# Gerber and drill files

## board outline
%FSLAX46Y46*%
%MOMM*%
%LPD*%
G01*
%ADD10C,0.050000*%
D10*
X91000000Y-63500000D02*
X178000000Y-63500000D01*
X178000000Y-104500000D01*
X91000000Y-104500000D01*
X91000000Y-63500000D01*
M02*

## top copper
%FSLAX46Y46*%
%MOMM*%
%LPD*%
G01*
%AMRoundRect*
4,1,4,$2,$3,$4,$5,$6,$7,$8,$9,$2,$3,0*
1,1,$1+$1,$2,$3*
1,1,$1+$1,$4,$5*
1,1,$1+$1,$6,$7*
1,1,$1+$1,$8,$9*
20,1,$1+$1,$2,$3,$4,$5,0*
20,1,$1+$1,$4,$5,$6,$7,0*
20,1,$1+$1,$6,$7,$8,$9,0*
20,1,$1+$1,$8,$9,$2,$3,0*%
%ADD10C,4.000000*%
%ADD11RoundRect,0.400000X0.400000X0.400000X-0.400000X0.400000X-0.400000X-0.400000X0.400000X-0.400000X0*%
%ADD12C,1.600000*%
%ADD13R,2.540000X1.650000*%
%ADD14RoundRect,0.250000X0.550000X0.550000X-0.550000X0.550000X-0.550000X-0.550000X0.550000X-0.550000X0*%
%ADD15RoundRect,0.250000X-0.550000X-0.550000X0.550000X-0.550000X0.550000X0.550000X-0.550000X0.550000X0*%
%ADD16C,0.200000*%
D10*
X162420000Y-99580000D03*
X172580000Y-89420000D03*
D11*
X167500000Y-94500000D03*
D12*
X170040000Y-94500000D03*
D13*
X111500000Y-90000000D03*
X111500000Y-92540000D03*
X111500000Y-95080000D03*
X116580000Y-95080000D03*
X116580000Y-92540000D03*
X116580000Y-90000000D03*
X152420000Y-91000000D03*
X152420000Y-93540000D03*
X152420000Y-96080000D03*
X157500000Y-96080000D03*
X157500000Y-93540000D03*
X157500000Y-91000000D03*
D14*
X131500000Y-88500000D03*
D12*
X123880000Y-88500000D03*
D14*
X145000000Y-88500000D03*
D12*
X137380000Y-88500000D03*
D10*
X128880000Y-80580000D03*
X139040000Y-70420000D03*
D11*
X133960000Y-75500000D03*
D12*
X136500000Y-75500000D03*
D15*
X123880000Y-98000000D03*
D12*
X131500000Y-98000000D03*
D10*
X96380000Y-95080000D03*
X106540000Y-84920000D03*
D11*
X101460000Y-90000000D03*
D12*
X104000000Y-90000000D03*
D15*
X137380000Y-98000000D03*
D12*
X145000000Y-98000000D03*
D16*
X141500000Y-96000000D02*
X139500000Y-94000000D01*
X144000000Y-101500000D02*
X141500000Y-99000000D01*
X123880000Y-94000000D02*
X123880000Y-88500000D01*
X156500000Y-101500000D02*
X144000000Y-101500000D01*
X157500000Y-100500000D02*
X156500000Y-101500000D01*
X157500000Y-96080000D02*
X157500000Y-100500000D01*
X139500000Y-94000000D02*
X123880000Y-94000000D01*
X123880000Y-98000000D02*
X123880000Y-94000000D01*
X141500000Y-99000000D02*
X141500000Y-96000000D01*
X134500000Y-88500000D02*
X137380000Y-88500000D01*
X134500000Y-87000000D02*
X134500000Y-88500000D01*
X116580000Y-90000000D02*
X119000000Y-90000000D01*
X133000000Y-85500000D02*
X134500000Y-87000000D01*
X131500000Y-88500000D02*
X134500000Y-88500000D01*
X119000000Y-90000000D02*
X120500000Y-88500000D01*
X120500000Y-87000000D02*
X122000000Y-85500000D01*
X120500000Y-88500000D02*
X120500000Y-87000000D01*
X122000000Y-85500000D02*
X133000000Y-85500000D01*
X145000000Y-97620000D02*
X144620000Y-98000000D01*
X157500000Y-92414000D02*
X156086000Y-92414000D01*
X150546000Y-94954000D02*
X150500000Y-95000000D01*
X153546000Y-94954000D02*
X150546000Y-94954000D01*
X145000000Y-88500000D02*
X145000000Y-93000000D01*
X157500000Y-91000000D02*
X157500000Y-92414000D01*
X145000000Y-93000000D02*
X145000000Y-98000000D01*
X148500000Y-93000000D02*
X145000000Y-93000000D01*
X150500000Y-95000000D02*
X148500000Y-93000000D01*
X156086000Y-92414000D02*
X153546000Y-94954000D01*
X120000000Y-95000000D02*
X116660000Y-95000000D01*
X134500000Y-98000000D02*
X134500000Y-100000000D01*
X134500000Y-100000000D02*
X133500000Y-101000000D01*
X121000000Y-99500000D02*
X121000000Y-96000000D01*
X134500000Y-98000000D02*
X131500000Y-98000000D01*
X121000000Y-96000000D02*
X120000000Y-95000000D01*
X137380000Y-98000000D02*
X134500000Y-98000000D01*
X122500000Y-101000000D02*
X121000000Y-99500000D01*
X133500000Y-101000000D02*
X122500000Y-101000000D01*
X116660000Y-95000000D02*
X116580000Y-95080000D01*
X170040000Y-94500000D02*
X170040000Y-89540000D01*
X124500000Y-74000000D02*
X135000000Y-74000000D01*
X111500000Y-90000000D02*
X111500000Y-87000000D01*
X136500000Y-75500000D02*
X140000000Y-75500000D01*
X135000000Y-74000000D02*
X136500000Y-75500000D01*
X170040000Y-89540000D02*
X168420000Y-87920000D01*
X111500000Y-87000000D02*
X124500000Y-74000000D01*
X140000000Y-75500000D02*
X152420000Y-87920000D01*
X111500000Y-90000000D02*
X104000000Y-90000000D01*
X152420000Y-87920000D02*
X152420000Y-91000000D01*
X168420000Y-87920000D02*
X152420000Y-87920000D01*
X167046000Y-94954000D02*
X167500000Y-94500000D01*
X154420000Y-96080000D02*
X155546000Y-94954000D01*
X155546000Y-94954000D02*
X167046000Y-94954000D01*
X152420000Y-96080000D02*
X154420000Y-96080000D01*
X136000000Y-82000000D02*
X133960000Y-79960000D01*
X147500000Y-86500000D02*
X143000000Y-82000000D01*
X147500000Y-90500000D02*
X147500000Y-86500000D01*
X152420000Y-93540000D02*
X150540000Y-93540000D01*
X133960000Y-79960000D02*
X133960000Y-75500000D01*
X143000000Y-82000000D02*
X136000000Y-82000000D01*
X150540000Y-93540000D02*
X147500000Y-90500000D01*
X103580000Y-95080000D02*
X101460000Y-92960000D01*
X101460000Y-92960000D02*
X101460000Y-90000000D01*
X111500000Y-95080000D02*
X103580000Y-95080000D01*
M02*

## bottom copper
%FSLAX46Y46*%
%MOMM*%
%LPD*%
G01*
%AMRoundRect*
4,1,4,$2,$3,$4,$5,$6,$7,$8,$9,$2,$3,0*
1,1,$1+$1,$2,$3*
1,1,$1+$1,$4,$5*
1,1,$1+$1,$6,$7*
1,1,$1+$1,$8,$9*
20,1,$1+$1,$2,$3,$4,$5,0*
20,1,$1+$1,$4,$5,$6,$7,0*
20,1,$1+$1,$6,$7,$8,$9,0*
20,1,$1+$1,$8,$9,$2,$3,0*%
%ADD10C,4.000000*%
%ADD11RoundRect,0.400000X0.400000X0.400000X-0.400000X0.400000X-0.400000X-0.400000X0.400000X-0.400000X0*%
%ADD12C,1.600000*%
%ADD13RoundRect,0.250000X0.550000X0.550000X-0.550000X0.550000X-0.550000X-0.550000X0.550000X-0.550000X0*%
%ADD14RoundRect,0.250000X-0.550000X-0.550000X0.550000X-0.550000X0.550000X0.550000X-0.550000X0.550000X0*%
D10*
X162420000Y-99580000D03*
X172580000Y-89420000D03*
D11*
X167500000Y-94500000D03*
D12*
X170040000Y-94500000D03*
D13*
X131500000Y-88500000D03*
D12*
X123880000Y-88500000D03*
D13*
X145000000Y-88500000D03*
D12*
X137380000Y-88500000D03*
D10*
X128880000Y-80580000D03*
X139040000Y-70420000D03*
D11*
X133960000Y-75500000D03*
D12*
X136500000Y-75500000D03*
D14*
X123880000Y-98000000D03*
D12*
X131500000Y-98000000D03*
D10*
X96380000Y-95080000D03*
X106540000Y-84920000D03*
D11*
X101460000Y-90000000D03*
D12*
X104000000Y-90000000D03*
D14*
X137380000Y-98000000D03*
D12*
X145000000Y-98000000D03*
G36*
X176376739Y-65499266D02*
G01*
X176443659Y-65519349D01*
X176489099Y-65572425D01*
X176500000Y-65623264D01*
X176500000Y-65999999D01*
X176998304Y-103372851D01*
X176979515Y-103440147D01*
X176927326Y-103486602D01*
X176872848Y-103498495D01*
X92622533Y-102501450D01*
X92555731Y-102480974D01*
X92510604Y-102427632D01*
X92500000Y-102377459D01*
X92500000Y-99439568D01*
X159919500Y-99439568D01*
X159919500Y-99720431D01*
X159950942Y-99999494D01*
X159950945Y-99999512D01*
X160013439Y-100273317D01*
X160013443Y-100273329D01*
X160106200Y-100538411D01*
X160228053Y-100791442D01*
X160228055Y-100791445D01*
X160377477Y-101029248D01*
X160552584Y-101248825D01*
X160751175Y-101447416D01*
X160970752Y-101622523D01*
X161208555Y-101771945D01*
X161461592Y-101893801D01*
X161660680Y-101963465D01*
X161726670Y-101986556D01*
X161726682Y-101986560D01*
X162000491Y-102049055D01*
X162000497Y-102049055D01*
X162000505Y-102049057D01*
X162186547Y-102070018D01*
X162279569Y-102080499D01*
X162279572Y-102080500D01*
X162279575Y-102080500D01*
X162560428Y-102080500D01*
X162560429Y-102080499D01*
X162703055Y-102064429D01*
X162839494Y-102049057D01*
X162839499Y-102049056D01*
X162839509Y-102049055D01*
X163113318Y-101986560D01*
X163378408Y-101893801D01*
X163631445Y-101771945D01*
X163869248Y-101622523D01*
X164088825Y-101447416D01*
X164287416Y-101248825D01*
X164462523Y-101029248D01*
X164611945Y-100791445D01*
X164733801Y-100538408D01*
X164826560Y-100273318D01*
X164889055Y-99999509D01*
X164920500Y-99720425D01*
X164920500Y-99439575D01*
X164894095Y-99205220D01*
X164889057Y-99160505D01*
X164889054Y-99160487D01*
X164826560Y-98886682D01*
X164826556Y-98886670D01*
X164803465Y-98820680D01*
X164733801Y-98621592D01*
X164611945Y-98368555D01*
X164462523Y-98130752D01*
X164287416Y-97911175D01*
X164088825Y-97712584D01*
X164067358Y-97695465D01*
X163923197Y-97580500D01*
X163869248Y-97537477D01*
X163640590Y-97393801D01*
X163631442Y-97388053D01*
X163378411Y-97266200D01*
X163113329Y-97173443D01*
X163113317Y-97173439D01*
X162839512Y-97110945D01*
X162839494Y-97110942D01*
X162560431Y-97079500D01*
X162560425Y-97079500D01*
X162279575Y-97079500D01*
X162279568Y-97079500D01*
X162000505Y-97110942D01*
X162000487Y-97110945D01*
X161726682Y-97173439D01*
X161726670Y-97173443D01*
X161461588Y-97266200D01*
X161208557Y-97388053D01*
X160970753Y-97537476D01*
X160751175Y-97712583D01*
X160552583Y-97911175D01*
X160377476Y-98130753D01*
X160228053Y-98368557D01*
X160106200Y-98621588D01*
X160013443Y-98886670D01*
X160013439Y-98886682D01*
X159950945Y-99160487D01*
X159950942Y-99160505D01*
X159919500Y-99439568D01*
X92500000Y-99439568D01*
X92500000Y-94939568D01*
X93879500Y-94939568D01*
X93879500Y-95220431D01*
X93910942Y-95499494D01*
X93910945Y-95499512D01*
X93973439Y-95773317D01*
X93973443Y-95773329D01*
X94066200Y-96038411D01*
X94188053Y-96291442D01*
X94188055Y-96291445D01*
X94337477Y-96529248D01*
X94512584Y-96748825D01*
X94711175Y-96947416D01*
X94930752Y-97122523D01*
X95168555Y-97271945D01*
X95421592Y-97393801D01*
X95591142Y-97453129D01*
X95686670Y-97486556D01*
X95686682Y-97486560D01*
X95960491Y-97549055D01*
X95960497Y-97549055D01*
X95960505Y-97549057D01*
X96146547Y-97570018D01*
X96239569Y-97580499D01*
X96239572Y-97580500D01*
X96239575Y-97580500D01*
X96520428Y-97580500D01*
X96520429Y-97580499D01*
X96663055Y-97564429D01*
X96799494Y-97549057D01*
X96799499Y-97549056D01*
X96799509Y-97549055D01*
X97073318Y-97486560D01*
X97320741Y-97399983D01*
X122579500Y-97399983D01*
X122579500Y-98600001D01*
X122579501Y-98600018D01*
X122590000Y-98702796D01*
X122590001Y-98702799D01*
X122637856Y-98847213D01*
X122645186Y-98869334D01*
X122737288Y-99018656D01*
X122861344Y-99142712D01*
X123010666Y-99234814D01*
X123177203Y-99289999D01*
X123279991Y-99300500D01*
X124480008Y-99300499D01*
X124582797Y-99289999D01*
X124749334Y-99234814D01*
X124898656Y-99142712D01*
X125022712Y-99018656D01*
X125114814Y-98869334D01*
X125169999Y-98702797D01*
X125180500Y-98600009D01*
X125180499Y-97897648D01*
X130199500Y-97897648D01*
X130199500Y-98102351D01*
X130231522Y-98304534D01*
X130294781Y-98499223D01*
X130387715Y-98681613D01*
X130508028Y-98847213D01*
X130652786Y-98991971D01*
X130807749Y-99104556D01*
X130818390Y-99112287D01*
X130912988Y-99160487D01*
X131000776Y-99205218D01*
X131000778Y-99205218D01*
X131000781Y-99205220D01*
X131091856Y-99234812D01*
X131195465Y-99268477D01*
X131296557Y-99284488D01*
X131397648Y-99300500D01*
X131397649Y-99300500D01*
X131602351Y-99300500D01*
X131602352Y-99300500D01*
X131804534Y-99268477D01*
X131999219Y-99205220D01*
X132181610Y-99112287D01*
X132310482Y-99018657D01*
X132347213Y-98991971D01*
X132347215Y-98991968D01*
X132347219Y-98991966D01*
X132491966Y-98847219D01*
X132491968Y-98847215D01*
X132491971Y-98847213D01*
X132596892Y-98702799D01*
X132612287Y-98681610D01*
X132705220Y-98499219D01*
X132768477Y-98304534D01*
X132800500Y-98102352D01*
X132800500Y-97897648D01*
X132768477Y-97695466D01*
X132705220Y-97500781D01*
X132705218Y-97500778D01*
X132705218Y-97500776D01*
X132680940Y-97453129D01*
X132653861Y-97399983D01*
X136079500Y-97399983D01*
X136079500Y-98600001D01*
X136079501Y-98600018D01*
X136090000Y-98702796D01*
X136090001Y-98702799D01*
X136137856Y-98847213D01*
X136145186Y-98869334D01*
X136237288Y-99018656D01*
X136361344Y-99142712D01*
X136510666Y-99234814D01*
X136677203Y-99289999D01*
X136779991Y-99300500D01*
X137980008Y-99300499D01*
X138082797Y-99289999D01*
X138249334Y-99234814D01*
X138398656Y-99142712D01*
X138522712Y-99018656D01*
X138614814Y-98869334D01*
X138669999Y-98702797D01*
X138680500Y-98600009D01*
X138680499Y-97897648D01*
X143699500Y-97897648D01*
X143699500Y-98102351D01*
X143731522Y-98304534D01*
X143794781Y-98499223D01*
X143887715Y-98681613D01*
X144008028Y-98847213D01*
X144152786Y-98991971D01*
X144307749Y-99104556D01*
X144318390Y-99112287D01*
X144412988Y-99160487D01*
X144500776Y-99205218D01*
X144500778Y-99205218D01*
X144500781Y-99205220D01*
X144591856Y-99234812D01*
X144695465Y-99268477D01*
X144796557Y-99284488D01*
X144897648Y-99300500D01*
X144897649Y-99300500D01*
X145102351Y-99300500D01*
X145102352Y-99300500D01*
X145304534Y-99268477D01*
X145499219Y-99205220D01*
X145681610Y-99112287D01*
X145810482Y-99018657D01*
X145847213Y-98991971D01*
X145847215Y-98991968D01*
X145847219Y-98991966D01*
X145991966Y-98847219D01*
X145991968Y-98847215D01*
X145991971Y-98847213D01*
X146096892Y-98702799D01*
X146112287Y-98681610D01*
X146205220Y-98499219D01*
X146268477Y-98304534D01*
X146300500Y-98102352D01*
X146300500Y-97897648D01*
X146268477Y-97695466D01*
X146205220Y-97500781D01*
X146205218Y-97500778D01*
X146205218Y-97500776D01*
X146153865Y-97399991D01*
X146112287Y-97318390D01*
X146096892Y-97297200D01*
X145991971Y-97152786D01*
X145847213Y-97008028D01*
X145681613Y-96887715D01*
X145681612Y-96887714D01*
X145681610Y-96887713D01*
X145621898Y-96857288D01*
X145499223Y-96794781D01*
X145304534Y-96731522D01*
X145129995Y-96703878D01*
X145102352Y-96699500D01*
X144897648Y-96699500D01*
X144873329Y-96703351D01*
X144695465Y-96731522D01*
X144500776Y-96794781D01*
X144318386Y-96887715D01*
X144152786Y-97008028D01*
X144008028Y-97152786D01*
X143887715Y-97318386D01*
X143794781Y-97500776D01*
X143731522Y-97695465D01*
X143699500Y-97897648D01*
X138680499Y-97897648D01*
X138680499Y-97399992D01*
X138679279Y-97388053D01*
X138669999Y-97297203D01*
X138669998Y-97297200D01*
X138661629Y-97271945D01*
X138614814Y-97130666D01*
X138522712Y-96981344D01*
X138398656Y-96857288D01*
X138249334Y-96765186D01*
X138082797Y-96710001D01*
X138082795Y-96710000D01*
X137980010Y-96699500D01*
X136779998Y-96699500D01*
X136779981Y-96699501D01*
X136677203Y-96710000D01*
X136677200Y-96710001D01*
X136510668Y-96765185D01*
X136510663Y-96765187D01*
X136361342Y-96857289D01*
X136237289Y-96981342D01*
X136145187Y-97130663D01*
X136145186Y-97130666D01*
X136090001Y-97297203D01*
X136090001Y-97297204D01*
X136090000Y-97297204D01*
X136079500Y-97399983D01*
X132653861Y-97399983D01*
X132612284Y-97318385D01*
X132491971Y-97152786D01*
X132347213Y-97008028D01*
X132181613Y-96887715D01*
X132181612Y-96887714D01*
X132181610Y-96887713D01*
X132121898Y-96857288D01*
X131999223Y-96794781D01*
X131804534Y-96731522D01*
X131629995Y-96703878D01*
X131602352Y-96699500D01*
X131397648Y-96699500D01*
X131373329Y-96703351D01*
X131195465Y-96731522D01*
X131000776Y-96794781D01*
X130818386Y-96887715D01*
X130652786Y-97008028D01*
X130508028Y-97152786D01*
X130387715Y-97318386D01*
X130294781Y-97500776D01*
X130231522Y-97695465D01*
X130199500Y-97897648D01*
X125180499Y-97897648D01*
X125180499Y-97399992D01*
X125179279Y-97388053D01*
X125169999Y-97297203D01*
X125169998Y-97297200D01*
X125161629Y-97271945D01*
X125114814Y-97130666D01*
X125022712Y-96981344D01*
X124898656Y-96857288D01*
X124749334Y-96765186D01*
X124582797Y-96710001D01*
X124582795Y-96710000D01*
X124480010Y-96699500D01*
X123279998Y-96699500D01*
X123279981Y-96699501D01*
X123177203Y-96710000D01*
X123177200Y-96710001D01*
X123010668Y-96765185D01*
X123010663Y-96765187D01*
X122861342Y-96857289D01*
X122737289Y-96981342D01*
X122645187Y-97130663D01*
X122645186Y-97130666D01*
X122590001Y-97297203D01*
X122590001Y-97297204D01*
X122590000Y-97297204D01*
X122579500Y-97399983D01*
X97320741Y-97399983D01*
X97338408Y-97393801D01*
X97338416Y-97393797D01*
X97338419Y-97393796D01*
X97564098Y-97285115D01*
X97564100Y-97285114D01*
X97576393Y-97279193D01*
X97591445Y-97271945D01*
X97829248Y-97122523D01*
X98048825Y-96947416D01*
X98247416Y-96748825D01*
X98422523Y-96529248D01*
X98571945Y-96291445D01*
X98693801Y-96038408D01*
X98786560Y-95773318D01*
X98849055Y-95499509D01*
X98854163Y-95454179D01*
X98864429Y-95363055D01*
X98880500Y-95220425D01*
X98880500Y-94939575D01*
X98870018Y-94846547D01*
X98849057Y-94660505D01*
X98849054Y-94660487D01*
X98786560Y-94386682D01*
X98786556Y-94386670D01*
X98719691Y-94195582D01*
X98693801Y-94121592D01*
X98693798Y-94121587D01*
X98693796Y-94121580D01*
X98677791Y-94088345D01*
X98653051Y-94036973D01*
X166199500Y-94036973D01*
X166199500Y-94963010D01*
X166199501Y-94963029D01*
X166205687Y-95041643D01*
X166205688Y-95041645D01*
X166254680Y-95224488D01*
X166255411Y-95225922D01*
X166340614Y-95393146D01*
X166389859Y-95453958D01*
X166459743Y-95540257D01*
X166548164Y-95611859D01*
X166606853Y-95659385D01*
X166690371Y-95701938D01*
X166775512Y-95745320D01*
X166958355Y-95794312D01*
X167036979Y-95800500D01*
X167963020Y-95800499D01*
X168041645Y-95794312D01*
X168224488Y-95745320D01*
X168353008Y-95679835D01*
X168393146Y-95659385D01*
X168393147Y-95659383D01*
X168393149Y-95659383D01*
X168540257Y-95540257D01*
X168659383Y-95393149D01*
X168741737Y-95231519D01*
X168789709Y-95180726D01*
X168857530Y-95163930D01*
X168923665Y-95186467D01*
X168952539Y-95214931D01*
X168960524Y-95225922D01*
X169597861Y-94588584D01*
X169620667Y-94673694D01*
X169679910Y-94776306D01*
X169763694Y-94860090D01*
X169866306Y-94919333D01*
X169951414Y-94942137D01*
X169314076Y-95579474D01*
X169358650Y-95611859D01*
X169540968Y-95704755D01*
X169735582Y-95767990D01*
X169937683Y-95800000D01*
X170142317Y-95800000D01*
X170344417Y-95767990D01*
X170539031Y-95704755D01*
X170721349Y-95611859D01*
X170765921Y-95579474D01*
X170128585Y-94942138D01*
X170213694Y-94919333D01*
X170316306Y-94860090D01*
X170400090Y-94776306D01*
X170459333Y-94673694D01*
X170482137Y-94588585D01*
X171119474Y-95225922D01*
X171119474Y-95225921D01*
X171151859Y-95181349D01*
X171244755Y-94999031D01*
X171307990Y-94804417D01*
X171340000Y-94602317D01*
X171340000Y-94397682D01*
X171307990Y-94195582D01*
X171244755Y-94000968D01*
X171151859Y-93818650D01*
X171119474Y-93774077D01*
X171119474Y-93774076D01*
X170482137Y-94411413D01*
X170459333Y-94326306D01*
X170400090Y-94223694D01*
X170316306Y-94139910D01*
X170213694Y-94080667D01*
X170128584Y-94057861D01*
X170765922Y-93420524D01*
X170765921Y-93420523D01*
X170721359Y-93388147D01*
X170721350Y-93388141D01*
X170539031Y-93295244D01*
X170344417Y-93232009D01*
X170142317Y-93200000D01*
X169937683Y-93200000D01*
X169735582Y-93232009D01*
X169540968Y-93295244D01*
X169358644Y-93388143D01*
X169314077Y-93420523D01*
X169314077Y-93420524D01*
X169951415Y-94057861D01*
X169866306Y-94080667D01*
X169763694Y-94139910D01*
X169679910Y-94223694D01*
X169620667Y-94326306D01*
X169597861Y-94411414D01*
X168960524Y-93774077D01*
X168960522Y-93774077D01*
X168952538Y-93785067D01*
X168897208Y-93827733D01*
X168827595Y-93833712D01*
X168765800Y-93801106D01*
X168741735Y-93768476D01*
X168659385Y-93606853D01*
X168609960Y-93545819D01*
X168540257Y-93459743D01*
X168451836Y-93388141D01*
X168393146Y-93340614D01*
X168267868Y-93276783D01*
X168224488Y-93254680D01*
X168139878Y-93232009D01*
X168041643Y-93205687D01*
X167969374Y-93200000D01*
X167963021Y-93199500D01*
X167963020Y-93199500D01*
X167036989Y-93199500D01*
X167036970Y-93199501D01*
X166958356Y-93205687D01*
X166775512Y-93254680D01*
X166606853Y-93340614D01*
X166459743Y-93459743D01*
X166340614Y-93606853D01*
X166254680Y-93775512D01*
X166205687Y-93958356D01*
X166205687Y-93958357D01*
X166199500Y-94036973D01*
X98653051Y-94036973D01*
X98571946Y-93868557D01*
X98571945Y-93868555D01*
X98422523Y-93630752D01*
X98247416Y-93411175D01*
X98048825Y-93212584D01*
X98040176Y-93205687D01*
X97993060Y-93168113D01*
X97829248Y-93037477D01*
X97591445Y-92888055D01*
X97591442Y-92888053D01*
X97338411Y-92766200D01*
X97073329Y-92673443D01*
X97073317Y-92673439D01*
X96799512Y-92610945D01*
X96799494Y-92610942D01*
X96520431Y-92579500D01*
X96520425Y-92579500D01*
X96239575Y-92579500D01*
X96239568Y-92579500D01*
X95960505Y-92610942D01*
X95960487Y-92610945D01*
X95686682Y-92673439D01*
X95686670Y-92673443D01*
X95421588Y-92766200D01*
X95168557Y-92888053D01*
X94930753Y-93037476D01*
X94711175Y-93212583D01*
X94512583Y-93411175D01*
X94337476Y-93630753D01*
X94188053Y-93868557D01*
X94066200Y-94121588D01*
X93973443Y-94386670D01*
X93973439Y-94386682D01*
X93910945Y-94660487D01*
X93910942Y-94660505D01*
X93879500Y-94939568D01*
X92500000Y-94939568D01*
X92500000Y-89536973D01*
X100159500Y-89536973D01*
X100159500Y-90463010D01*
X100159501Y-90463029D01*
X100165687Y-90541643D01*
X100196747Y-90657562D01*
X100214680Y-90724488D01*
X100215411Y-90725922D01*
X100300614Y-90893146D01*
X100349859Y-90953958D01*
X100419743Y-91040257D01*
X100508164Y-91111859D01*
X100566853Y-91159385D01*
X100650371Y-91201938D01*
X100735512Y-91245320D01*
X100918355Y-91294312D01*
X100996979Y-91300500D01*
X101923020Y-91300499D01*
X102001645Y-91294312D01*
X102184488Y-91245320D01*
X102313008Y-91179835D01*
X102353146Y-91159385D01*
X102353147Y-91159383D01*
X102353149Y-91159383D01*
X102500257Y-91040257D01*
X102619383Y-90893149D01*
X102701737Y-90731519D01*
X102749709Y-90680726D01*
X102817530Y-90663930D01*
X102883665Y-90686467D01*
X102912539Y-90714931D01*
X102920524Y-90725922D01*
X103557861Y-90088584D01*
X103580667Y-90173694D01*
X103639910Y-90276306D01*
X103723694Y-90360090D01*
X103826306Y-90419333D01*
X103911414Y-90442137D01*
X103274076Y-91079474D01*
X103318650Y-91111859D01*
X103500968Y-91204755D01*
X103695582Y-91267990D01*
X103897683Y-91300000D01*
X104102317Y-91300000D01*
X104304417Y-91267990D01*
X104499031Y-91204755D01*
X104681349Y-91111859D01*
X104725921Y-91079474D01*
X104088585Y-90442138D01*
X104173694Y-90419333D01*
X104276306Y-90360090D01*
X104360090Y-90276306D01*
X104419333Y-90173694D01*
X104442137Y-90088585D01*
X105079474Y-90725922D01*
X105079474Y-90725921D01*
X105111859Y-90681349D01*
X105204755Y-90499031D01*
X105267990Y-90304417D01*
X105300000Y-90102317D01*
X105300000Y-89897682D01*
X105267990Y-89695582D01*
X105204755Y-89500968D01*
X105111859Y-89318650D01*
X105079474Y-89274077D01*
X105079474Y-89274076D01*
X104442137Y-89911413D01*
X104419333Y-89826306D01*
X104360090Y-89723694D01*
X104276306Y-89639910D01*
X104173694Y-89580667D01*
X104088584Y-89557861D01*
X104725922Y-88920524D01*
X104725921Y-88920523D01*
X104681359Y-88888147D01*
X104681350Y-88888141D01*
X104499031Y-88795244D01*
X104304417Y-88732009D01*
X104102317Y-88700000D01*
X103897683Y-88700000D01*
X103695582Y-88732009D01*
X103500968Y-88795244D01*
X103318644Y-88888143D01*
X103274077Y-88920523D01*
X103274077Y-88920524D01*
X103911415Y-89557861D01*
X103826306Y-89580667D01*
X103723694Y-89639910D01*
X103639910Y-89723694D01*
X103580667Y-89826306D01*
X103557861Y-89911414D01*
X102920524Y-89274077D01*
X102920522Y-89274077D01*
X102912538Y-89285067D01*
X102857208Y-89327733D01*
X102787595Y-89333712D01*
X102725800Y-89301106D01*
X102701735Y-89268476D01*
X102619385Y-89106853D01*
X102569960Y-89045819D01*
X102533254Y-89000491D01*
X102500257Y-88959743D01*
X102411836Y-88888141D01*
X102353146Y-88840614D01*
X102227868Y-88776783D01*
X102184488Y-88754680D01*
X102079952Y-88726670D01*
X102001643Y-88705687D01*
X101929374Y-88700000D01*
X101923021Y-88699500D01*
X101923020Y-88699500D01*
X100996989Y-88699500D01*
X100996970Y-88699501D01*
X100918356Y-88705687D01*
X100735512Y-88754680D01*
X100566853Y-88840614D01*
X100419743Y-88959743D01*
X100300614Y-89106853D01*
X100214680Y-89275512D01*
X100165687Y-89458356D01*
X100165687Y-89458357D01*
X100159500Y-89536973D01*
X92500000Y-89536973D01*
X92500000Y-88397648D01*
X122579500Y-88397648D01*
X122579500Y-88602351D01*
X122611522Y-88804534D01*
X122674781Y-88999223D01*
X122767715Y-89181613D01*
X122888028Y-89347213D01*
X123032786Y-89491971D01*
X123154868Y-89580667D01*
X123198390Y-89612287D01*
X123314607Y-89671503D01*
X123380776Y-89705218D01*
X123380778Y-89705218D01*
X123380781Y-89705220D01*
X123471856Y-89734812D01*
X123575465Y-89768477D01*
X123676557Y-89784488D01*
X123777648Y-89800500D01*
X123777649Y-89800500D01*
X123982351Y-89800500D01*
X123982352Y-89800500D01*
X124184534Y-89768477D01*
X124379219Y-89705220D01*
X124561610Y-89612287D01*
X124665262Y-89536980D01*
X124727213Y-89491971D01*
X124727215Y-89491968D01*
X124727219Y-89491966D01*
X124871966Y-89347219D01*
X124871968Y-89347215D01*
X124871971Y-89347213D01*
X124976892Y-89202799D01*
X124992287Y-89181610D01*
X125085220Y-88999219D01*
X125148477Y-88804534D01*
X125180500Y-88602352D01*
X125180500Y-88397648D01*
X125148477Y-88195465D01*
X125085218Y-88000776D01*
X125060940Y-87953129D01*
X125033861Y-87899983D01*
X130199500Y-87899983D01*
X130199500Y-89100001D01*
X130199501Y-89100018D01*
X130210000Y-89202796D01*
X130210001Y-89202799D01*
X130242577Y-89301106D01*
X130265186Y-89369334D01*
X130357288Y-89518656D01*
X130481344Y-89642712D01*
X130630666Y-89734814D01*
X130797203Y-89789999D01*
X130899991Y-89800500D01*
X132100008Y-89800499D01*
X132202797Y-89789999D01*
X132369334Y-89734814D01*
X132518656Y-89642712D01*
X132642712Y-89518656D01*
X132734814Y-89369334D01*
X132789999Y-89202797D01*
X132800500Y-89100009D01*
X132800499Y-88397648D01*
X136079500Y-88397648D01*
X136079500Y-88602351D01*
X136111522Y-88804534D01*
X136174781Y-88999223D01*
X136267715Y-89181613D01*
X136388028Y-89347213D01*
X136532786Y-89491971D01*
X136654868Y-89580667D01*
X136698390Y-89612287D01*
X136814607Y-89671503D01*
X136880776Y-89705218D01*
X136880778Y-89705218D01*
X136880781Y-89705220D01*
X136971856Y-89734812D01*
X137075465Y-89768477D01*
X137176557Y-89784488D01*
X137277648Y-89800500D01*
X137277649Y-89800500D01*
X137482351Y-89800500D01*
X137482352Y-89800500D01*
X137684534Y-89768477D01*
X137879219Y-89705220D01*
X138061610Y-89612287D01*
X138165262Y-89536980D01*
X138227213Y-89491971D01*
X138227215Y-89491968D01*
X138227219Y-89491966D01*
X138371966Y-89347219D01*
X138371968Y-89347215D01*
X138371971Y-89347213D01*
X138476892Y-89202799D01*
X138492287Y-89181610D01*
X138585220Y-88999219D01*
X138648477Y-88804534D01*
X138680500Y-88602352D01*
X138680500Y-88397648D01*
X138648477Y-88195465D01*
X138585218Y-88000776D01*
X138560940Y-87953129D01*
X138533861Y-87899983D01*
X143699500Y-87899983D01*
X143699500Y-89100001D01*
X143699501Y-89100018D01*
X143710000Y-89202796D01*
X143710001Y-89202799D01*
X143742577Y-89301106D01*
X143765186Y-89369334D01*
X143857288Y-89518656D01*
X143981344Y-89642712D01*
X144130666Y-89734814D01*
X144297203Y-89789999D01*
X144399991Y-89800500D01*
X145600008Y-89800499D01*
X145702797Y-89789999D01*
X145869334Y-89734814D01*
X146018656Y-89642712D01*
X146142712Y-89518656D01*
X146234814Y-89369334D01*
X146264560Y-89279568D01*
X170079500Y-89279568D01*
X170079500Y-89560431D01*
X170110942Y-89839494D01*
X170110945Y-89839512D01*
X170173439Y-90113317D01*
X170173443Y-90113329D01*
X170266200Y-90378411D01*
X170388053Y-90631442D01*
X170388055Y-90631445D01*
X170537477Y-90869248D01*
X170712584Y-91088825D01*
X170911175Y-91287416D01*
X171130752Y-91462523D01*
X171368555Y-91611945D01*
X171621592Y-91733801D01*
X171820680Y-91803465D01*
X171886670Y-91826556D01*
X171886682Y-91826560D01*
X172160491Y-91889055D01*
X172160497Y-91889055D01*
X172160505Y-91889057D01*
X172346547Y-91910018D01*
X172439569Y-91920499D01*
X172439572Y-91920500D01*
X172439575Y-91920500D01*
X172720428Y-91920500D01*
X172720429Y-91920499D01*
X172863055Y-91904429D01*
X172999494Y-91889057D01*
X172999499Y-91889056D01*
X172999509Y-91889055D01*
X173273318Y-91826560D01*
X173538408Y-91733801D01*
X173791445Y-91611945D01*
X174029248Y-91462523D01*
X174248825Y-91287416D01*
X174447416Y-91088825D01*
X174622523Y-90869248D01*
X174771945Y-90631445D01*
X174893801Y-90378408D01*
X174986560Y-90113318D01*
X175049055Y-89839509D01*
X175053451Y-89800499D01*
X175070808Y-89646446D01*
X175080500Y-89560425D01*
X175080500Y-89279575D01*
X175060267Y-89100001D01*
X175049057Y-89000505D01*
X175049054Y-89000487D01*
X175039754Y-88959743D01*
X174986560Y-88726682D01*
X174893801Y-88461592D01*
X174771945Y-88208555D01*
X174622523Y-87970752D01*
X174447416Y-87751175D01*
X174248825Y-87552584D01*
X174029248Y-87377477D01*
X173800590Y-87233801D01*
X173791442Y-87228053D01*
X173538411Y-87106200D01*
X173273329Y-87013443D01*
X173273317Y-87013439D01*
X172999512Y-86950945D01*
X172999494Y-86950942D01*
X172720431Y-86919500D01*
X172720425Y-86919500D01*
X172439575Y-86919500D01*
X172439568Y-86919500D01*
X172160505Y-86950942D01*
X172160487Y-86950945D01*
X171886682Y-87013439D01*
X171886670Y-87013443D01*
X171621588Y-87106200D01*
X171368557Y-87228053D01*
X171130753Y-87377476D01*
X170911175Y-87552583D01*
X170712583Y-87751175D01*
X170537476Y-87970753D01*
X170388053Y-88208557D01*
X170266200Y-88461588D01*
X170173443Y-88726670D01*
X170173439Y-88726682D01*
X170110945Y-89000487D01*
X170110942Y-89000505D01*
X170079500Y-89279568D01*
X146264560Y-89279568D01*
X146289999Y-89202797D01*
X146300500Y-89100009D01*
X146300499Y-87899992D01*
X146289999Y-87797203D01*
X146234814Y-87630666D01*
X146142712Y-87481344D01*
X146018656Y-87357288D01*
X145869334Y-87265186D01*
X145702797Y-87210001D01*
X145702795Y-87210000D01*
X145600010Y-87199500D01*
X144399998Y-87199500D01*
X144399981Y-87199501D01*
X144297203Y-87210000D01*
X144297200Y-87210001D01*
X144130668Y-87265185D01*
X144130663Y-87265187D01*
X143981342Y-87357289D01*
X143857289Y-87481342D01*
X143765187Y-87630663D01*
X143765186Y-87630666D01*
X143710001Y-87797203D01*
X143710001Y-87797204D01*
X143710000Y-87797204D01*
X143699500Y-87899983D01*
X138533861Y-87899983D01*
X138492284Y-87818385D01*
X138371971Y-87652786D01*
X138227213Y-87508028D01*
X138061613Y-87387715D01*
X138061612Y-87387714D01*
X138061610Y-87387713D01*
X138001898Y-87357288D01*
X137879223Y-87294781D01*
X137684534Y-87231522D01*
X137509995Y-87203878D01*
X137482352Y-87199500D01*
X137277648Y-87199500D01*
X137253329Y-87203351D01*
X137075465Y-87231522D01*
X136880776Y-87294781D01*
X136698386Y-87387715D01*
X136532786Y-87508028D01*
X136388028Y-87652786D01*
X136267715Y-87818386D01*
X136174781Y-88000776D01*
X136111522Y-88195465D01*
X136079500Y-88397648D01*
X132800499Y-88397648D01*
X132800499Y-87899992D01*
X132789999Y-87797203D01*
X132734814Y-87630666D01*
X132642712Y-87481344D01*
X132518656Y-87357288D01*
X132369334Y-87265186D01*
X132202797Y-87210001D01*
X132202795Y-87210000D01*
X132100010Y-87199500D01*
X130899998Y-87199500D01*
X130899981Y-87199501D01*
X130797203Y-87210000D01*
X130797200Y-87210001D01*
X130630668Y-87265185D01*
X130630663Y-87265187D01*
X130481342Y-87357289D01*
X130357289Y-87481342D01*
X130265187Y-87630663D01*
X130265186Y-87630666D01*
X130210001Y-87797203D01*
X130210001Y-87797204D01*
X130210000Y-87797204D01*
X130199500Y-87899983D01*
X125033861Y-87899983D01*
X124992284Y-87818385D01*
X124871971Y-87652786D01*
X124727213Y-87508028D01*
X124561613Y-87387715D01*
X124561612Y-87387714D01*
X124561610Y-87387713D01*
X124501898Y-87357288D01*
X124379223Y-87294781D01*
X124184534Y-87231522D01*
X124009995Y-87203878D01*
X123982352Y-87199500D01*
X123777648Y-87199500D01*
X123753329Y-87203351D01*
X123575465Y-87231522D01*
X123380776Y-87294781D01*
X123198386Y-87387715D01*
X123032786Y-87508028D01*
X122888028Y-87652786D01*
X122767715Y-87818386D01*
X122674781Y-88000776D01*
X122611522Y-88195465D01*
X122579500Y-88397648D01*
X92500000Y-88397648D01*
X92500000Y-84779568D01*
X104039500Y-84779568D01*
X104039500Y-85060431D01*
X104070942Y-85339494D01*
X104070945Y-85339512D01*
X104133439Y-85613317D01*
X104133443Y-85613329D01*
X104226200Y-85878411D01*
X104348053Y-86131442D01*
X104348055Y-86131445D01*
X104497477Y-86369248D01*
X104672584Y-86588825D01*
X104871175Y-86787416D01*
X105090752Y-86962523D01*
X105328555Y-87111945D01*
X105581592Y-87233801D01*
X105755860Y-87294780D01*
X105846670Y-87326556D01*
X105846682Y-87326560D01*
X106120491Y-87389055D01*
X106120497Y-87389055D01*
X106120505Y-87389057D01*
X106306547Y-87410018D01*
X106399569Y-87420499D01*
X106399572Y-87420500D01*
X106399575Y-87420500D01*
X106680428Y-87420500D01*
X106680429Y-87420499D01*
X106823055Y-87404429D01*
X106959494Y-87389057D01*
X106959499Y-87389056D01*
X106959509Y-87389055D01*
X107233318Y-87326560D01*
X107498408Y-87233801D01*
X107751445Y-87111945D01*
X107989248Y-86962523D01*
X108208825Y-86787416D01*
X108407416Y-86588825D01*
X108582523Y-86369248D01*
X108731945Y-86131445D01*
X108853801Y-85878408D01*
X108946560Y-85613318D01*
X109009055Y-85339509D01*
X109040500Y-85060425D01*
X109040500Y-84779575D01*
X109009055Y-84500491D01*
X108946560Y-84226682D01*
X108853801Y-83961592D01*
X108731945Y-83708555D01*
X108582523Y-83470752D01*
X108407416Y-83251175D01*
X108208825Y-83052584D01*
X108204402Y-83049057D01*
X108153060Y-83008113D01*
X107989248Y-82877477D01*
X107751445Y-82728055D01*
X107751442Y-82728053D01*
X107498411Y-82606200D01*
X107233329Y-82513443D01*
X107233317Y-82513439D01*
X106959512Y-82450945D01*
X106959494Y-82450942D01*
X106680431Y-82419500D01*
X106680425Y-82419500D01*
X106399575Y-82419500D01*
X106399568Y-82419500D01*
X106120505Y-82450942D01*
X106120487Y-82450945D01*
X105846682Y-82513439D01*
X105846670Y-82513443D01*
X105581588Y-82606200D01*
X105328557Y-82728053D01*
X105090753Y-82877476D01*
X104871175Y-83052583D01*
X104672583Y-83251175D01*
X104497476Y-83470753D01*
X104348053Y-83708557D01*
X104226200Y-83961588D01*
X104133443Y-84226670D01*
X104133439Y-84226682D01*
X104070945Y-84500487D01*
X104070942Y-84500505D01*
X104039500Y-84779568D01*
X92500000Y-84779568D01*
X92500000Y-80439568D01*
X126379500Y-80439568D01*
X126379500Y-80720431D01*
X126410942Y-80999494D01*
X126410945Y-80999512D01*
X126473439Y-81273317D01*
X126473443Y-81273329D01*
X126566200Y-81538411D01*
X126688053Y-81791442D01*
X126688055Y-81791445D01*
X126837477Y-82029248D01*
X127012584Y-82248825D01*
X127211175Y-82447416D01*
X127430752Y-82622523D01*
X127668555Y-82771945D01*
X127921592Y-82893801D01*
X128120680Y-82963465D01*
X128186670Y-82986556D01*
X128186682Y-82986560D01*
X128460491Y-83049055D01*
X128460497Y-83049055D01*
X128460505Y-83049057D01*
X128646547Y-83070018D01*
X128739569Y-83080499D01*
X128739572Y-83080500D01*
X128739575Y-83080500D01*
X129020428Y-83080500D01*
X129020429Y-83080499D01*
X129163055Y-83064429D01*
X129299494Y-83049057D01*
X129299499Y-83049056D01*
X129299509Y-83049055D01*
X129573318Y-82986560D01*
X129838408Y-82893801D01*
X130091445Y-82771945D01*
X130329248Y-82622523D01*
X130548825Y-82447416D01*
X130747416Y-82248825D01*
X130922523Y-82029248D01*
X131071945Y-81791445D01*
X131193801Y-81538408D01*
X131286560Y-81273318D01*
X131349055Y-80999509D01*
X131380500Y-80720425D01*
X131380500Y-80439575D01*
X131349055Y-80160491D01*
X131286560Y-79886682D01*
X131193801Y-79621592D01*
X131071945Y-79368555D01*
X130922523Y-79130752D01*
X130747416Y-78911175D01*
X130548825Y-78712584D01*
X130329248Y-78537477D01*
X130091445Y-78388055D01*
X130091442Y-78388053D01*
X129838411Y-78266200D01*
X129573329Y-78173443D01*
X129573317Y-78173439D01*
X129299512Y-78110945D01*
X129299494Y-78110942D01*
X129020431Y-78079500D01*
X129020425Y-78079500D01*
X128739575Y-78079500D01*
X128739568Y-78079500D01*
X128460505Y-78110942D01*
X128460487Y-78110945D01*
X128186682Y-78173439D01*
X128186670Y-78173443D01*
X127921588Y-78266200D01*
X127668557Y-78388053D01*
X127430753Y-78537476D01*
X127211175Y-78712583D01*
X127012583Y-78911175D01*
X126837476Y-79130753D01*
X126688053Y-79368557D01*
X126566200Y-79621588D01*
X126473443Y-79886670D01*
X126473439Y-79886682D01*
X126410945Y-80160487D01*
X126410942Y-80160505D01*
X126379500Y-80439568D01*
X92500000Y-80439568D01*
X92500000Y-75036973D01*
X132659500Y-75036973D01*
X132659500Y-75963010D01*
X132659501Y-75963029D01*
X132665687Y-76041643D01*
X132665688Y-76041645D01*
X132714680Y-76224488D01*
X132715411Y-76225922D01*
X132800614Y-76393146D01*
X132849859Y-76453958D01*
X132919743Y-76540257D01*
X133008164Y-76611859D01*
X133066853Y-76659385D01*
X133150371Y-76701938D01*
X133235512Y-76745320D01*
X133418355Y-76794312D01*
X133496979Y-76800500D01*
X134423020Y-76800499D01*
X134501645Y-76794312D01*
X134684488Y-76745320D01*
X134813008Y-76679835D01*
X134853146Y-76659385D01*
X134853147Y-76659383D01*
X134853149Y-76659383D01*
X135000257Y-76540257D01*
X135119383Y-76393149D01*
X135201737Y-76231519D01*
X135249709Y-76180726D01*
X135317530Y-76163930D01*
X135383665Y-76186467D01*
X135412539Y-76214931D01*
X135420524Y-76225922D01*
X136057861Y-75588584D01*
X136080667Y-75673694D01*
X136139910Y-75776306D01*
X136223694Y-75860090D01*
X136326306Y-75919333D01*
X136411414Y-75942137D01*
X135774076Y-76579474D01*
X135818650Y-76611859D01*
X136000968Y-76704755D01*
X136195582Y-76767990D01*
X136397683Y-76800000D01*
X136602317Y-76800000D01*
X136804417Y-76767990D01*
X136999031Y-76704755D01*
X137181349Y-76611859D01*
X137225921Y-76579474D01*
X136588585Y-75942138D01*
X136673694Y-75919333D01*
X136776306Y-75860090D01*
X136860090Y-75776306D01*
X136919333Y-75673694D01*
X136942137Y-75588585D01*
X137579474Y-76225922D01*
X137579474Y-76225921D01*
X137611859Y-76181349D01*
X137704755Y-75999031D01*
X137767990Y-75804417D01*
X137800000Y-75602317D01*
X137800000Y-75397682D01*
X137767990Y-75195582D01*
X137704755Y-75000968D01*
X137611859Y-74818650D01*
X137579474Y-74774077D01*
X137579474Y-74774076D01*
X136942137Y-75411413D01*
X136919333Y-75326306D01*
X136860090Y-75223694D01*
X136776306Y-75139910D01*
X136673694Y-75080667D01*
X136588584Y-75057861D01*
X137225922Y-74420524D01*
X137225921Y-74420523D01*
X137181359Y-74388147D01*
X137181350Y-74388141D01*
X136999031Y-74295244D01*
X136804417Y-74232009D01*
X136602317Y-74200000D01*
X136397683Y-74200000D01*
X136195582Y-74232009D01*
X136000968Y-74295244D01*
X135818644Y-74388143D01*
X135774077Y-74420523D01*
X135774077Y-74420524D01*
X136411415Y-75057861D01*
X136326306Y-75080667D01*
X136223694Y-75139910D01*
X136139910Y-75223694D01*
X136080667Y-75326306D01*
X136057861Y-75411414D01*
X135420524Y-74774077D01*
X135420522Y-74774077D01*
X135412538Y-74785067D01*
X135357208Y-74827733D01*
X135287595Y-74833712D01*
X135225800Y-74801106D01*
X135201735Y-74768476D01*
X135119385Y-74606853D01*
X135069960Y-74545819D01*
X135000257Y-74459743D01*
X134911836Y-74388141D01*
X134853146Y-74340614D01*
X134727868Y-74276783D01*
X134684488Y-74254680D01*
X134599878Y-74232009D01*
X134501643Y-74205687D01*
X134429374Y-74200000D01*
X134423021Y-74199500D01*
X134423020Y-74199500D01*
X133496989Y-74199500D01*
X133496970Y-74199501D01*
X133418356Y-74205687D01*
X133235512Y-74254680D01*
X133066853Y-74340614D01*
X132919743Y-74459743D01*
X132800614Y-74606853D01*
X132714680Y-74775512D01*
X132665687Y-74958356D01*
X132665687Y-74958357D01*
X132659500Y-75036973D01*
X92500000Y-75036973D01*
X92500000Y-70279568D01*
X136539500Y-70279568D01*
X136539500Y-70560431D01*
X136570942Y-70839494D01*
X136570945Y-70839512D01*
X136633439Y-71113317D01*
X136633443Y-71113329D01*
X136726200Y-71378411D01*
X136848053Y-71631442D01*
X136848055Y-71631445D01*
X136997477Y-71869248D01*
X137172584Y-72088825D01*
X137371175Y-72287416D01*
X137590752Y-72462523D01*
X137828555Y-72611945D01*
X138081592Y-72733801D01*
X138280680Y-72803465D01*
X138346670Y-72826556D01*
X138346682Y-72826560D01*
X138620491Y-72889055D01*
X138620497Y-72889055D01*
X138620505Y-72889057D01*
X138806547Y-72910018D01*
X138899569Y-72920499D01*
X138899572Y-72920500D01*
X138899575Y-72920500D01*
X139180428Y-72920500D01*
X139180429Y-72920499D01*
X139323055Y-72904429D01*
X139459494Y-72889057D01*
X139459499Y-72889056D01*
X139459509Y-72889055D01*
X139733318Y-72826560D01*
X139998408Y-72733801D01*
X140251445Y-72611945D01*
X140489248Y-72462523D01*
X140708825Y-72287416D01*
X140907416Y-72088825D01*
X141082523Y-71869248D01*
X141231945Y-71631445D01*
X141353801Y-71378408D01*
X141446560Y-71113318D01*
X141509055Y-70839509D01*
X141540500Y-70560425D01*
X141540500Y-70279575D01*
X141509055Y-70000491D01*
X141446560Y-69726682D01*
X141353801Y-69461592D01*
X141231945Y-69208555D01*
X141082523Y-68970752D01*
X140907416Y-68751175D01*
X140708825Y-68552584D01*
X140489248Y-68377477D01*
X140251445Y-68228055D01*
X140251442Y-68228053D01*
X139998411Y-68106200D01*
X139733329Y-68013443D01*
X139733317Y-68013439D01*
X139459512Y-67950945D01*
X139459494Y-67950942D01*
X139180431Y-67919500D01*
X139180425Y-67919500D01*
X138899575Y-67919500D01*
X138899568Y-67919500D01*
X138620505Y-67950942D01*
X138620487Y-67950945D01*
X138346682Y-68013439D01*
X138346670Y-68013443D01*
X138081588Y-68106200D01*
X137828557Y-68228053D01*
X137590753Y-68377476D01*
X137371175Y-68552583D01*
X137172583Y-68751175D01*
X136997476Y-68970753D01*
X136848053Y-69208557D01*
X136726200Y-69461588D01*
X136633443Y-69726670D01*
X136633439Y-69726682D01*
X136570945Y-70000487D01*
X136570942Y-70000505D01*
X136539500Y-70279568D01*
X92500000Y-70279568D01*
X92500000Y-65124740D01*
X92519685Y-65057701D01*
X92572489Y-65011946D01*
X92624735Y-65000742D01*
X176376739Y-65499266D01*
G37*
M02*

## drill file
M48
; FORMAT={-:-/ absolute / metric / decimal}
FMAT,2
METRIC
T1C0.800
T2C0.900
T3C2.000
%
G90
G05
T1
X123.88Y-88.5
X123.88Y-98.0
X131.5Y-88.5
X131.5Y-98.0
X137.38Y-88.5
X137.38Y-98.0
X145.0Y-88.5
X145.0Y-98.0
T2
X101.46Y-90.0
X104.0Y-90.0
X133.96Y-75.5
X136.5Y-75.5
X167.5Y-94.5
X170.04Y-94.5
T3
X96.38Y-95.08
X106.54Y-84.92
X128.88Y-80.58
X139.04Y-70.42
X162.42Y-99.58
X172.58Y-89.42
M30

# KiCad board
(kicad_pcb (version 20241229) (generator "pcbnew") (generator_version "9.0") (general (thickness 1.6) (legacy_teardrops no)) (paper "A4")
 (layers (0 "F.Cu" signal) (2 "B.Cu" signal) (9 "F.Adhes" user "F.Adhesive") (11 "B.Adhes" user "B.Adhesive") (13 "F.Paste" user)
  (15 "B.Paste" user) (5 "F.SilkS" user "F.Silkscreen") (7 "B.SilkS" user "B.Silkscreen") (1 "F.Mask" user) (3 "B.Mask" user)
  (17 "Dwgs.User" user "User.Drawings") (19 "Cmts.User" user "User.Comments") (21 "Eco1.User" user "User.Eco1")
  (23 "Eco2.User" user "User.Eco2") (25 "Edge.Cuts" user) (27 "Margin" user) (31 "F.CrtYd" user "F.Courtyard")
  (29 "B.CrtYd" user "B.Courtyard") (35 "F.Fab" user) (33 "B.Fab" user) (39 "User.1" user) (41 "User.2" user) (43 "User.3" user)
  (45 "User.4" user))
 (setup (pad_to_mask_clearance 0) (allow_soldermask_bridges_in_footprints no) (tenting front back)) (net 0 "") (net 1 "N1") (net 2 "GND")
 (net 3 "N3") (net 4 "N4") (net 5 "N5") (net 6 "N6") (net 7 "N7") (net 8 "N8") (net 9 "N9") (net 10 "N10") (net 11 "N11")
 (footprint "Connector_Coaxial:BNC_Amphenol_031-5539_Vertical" (layer "F.Cu") (at 167.5 94.5)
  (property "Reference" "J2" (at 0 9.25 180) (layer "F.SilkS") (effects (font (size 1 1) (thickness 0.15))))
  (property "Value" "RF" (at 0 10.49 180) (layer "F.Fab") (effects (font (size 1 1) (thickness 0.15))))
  (pad "" thru_hole circle (at -5.08 5.08 180) (size 4 4) (drill 2) (layers "*.Cu" "*.Mask") (remove_unused_layers no))
  (pad "" thru_hole circle (at 5.08 -5.08 180) (size 4 4) (drill 2) (layers "*.Cu" "*.Mask") (remove_unused_layers no))
  (pad "1" thru_hole roundrect (at 0 0 180) (size 1.6 1.6) (drill 0.9) (layers "*.Cu" "*.Mask") (remove_unused_layers no)
   (roundrect_rratio 0.25) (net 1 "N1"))
  (pad "2" thru_hole circle (at 2.54 0 180) (size 1.6 1.6) (drill 0.9) (layers "*.Cu" "*.Mask") (remove_unused_layers no) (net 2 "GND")))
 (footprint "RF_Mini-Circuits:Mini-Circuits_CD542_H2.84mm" (layer "F.Cu") (at 114.04 92.54)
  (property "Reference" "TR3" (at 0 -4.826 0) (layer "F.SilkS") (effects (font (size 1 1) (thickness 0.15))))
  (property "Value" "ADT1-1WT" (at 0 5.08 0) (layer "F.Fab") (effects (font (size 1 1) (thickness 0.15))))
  (pad "1" smd rect (at -2.54 -2.54) (size 2.54 1.65) (layers "F.Cu" "F.Mask" "F.Paste") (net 2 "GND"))
  (pad "2" smd rect (at -2.54 0) (size 2.54 1.65) (layers "F.Cu" "F.Mask" "F.Paste") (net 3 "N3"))
  (pad "3" smd rect (at -2.54 2.54) (size 2.54 1.65) (layers "F.Cu" "F.Mask" "F.Paste") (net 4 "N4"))
  (pad "4" smd rect (at 2.54 2.54) (size 2.54 1.65) (layers "F.Cu" "F.Mask" "F.Paste") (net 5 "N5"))
  (pad "5" smd rect (at 2.54 0) (size 2.54 1.65) (layers "F.Cu" "F.Mask" "F.Paste") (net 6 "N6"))
  (pad "6" smd rect (at 2.54 -2.54) (size 2.54 1.65) (layers "F.Cu" "F.Mask" "F.Paste") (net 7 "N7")))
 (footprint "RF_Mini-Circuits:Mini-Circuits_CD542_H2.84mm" (layer "F.Cu") (at 154.96 93.54)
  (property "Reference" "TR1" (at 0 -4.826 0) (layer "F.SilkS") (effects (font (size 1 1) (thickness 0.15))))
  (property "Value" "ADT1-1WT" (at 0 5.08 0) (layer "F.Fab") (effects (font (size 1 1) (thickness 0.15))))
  (pad "1" smd rect (at -2.54 -2.54) (size 2.54 1.65) (layers "F.Cu" "F.Mask" "F.Paste") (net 2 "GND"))
  (pad "2" smd rect (at -2.54 0) (size 2.54 1.65) (layers "F.Cu" "F.Mask" "F.Paste") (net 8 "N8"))
  (pad "3" smd rect (at -2.54 2.54) (size 2.54 1.65) (layers "F.Cu" "F.Mask" "F.Paste") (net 1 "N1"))
  (pad "4" smd rect (at 2.54 2.54) (size 2.54 1.65) (layers "F.Cu" "F.Mask" "F.Paste") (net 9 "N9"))
  (pad "5" smd rect (at 2.54 0) (size 2.54 1.65) (layers "F.Cu" "F.Mask" "F.Paste") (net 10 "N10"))
  (pad "6" smd rect (at 2.54 -2.54) (size 2.54 1.65) (layers "F.Cu" "F.Mask" "F.Paste") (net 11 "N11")))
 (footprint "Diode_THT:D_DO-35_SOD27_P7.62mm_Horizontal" (layer "F.Cu") (at 131.5 88.5 180)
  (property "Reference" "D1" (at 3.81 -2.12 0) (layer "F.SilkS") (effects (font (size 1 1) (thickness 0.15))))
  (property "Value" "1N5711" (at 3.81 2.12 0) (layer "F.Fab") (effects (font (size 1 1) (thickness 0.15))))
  (pad "1" thru_hole roundrect (at 0 0 180) (size 1.6 1.6) (drill 0.8) (layers "*.Cu" "*.Mask") (remove_unused_layers no)
   (roundrect_rratio 0.15625) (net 7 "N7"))
  (pad "2" thru_hole circle (at 7.62 0 180) (size 1.6 1.6) (drill 0.8) (layers "*.Cu" "*.Mask") (remove_unused_layers no) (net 9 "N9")))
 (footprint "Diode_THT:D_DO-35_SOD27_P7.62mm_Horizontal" (layer "F.Cu") (at 145 88.5 180)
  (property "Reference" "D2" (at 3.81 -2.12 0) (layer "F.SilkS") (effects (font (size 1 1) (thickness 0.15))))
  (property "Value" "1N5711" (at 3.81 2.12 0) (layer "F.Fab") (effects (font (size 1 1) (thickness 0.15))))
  (pad "1" thru_hole roundrect (at 0 0 180) (size 1.6 1.6) (drill 0.8) (layers "*.Cu" "*.Mask") (remove_unused_layers no)
   (roundrect_rratio 0.15625) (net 11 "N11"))
  (pad "2" thru_hole circle (at 7.62 0 180) (size 1.6 1.6) (drill 0.8) (layers "*.Cu" "*.Mask") (remove_unused_layers no) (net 7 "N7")))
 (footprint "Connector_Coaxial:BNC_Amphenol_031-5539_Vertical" (layer "F.Cu") (at 133.96 75.5)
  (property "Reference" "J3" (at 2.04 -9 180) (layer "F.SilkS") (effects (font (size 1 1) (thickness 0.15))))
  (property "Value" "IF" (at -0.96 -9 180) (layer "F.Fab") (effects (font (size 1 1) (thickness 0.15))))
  (pad "" thru_hole circle (at -5.08 5.08 180) (size 4 4) (drill 2) (layers "*.Cu" "*.Mask") (remove_unused_layers no))
  (pad "" thru_hole circle (at 5.08 -5.08 180) (size 4 4) (drill 2) (layers "*.Cu" "*.Mask") (remove_unused_layers no))
  (pad "1" thru_hole roundrect (at 0 0 180) (size 1.6 1.6) (drill 0.9) (layers "*.Cu" "*.Mask") (remove_unused_layers no)
   (roundrect_rratio 0.25) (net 8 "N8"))
  (pad "2" thru_hole circle (at 2.54 0 180) (size 1.6 1.6) (drill 0.9) (layers "*.Cu" "*.Mask") (remove_unused_layers no) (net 2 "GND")))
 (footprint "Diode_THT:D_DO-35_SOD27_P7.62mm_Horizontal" (layer "F.Cu") (at 123.88 98)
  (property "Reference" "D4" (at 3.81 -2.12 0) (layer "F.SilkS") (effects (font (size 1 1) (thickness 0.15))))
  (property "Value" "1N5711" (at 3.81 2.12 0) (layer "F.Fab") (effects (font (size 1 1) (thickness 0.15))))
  (pad "1" thru_hole roundrect (at 0 0) (size 1.6 1.6) (drill 0.8) (layers "*.Cu" "*.Mask") (remove_unused_layers no)
   (roundrect_rratio 0.15625) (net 9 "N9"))
  (pad "2" thru_hole circle (at 7.62 0) (size 1.6 1.6) (drill 0.8) (layers "*.Cu" "*.Mask") (remove_unused_layers no) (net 5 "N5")))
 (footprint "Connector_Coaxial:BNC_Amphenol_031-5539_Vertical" (layer "F.Cu") (at 101.46 90)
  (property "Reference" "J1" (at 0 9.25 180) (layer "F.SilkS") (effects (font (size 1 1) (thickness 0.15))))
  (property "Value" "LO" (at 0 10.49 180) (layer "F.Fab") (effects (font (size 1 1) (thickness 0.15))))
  (pad "" thru_hole circle (at -5.08 5.08 180) (size 4 4) (drill 2) (layers "*.Cu" "*.Mask") (remove_unused_layers no))
  (pad "" thru_hole circle (at 5.08 -5.08 180) (size 4 4) (drill 2) (layers "*.Cu" "*.Mask") (remove_unused_layers no))
  (pad "1" thru_hole roundrect (at 0 0 180) (size 1.6 1.6) (drill 0.9) (layers "*.Cu" "*.Mask") (remove_unused_layers no)
   (roundrect_rratio 0.25) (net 4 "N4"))
  (pad "2" thru_hole circle (at 2.54 0 180) (size 1.6 1.6) (drill 0.9) (layers "*.Cu" "*.Mask") (remove_unused_layers no) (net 2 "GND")))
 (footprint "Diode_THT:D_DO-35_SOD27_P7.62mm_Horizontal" (layer "F.Cu") (at 137.38 98)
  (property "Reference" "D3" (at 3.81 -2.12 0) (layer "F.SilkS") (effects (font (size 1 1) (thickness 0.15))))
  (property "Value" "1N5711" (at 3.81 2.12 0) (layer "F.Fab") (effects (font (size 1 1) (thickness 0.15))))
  (pad "1" thru_hole roundrect (at 0 0) (size 1.6 1.6) (drill 0.8) (layers "*.Cu" "*.Mask") (remove_unused_layers no)
   (roundrect_rratio 0.15625) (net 5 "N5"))
  (pad "2" thru_hole circle (at 7.62 0) (size 1.6 1.6) (drill 0.8) (layers "*.Cu" "*.Mask") (remove_unused_layers no) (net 11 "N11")))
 (gr_rect (start 91 63.5) (end 178 104.5) (stroke (width 0.05) (type default)) (fill no) (layer "Edge.Cuts"))
 (segment (start 141.5 96) (end 139.5 94) (width 0.2) (layer "F.Cu") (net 9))
 (segment (start 144 101.5) (end 141.5 99) (width 0.2) (layer "F.Cu") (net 9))
 (segment (start 123.88 94) (end 123.88 88.5) (width 0.2) (layer "F.Cu") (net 9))
 (segment (start 156.5 101.5) (end 144 101.5) (width 0.2) (layer "F.Cu") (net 9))
 (segment (start 157.5 100.5) (end 156.5 101.5) (width 0.2) (layer "F.Cu") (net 9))
 (segment (start 157.5 96.08) (end 157.5 100.5) (width 0.2) (layer "F.Cu") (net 9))
 (segment (start 139.5 94) (end 123.88 94) (width 0.2) (layer "F.Cu") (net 9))
 (segment (start 123.88 98) (end 123.88 94) (width 0.2) (layer "F.Cu") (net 9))
 (segment (start 141.5 99) (end 141.5 96) (width 0.2) (layer "F.Cu") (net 9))
 (segment (start 134.5 88.5) (end 137.38 88.5) (width 0.2) (layer "F.Cu") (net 7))
 (segment (start 134.5 87) (end 134.5 88.5) (width 0.2) (layer "F.Cu") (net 7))
 (segment (start 116.58 90) (end 119 90) (width 0.2) (layer "F.Cu") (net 7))
 (segment (start 133 85.5) (end 134.5 87) (width 0.2) (layer "F.Cu") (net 7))
 (segment (start 131.5 88.5) (end 134.5 88.5) (width 0.2) (layer "F.Cu") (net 7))
 (segment (start 119 90) (end 120.5 88.5) (width 0.2) (layer "F.Cu") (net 7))
 (segment (start 120.5 87) (end 122 85.5) (width 0.2) (layer "F.Cu") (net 7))
 (segment (start 120.5 88.5) (end 120.5 87) (width 0.2) (layer "F.Cu") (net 7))
 (segment (start 122 85.5) (end 133 85.5) (width 0.2) (layer "F.Cu") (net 7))
 (segment (start 145 97.62) (end 144.62 98) (width 0.2) (layer "F.Cu") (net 11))
 (segment (start 157.5 92.414) (end 156.086 92.414) (width 0.2) (layer "F.Cu") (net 11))
 (segment (start 150.546 94.954) (end 150.5 95) (width 0.2) (layer "F.Cu") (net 11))
 (segment (start 153.546 94.954) (end 150.546 94.954) (width 0.2) (layer "F.Cu") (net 11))
 (segment (start 145 88.5) (end 145 93) (width 0.2) (layer "F.Cu") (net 11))
 (segment (start 157.5 91) (end 157.5 92.414) (width 0.2) (layer "F.Cu") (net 11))
 (segment (start 145 93) (end 145 98) (width 0.2) (layer "F.Cu") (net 11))
 (segment (start 148.5 93) (end 145 93) (width 0.2) (layer "F.Cu") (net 11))
 (segment (start 150.5 95) (end 148.5 93) (width 0.2) (layer "F.Cu") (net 11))
 (segment (start 156.086 92.414) (end 153.546 94.954) (width 0.2) (layer "F.Cu") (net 11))
 (segment (start 120 95) (end 116.66 95) (width 0.2) (layer "F.Cu") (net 5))
 (segment (start 134.5 98) (end 134.5 100) (width 0.2) (layer "F.Cu") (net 5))
 (segment (start 134.5 100) (end 133.5 101) (width 0.2) (layer "F.Cu") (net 5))
 (segment (start 121 99.5) (end 121 96) (width 0.2) (layer "F.Cu") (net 5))
 (segment (start 134.5 98) (end 131.5 98) (width 0.2) (layer "F.Cu") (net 5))
 (segment (start 121 96) (end 120 95) (width 0.2) (layer "F.Cu") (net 5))
 (segment (start 137.38 98) (end 134.5 98) (width 0.2) (layer "F.Cu") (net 5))
 (segment (start 122.5 101) (end 121 99.5) (width 0.2) (layer "F.Cu") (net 5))
 (segment (start 133.5 101) (end 122.5 101) (width 0.2) (layer "F.Cu") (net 5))
 (segment (start 116.66 95) (end 116.58 95.08) (width 0.2) (layer "F.Cu") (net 5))
 (segment (start 170.04 94.5) (end 170.04 89.54) (width 0.2) (layer "F.Cu") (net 2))
 (segment (start 124.5 74) (end 135 74) (width 0.2) (layer "F.Cu") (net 2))
 (segment (start 111.5 90) (end 111.5 87) (width 0.2) (layer "F.Cu") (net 2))
 (segment (start 136.5 75.5) (end 140 75.5) (width 0.2) (layer "F.Cu") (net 2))
 (segment (start 135 74) (end 136.5 75.5) (width 0.2) (layer "F.Cu") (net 2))
 (segment (start 170.04 89.54) (end 168.42 87.92) (width 0.2) (layer "F.Cu") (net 2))
 (segment (start 111.5 87) (end 124.5 74) (width 0.2) (layer "F.Cu") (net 2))
 (segment (start 140 75.5) (end 152.42 87.92) (width 0.2) (layer "F.Cu") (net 2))
 (segment (start 111.5 90) (end 104 90) (width 0.2) (layer "F.Cu") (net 2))
 (segment (start 152.42 87.92) (end 152.42 91) (width 0.2) (layer "F.Cu") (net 2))
 (segment (start 168.42 87.92) (end 152.42 87.92) (width 0.2) (layer "F.Cu") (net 2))
 (segment (start 167.046 94.954) (end 167.5 94.5) (width 0.2) (layer "F.Cu") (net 1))
 (segment (start 154.42 96.08) (end 155.546 94.954) (width 0.2) (layer "F.Cu") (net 1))
 (segment (start 155.546 94.954) (end 167.046 94.954) (width 0.2) (layer "F.Cu") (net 1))
 (segment (start 152.42 96.08) (end 154.42 96.08) (width 0.2) (layer "F.Cu") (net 1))
 (segment (start 136 82) (end 133.96 79.96) (width 0.2) (layer "F.Cu") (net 8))
 (segment (start 147.5 86.5) (end 143 82) (width 0.2) (layer "F.Cu") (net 8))
 (segment (start 147.5 90.5) (end 147.5 86.5) (width 0.2) (layer "F.Cu") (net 8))
 (segment (start 152.42 93.54) (end 150.54 93.54) (width 0.2) (layer "F.Cu") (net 8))
 (segment (start 133.96 79.96) (end 133.96 75.5) (width 0.2) (layer "F.Cu") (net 8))
 (segment (start 143 82) (end 136 82) (width 0.2) (layer "F.Cu") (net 8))
 (segment (start 150.54 93.54) (end 147.5 90.5) (width 0.2) (layer "F.Cu") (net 8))
 (segment (start 103.58 95.08) (end 101.46 92.96) (width 0.2) (layer "F.Cu") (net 4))
 (segment (start 101.46 92.96) (end 101.46 90) (width 0.2) (layer "F.Cu") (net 4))
 (segment (start 111.5 95.08) (end 103.58 95.08) (width 0.2) (layer "F.Cu") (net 4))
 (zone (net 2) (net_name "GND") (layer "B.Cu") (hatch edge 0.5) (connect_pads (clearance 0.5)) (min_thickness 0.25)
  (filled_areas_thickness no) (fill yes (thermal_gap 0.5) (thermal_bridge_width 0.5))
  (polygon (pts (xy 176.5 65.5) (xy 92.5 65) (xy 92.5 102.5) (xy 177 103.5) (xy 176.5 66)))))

